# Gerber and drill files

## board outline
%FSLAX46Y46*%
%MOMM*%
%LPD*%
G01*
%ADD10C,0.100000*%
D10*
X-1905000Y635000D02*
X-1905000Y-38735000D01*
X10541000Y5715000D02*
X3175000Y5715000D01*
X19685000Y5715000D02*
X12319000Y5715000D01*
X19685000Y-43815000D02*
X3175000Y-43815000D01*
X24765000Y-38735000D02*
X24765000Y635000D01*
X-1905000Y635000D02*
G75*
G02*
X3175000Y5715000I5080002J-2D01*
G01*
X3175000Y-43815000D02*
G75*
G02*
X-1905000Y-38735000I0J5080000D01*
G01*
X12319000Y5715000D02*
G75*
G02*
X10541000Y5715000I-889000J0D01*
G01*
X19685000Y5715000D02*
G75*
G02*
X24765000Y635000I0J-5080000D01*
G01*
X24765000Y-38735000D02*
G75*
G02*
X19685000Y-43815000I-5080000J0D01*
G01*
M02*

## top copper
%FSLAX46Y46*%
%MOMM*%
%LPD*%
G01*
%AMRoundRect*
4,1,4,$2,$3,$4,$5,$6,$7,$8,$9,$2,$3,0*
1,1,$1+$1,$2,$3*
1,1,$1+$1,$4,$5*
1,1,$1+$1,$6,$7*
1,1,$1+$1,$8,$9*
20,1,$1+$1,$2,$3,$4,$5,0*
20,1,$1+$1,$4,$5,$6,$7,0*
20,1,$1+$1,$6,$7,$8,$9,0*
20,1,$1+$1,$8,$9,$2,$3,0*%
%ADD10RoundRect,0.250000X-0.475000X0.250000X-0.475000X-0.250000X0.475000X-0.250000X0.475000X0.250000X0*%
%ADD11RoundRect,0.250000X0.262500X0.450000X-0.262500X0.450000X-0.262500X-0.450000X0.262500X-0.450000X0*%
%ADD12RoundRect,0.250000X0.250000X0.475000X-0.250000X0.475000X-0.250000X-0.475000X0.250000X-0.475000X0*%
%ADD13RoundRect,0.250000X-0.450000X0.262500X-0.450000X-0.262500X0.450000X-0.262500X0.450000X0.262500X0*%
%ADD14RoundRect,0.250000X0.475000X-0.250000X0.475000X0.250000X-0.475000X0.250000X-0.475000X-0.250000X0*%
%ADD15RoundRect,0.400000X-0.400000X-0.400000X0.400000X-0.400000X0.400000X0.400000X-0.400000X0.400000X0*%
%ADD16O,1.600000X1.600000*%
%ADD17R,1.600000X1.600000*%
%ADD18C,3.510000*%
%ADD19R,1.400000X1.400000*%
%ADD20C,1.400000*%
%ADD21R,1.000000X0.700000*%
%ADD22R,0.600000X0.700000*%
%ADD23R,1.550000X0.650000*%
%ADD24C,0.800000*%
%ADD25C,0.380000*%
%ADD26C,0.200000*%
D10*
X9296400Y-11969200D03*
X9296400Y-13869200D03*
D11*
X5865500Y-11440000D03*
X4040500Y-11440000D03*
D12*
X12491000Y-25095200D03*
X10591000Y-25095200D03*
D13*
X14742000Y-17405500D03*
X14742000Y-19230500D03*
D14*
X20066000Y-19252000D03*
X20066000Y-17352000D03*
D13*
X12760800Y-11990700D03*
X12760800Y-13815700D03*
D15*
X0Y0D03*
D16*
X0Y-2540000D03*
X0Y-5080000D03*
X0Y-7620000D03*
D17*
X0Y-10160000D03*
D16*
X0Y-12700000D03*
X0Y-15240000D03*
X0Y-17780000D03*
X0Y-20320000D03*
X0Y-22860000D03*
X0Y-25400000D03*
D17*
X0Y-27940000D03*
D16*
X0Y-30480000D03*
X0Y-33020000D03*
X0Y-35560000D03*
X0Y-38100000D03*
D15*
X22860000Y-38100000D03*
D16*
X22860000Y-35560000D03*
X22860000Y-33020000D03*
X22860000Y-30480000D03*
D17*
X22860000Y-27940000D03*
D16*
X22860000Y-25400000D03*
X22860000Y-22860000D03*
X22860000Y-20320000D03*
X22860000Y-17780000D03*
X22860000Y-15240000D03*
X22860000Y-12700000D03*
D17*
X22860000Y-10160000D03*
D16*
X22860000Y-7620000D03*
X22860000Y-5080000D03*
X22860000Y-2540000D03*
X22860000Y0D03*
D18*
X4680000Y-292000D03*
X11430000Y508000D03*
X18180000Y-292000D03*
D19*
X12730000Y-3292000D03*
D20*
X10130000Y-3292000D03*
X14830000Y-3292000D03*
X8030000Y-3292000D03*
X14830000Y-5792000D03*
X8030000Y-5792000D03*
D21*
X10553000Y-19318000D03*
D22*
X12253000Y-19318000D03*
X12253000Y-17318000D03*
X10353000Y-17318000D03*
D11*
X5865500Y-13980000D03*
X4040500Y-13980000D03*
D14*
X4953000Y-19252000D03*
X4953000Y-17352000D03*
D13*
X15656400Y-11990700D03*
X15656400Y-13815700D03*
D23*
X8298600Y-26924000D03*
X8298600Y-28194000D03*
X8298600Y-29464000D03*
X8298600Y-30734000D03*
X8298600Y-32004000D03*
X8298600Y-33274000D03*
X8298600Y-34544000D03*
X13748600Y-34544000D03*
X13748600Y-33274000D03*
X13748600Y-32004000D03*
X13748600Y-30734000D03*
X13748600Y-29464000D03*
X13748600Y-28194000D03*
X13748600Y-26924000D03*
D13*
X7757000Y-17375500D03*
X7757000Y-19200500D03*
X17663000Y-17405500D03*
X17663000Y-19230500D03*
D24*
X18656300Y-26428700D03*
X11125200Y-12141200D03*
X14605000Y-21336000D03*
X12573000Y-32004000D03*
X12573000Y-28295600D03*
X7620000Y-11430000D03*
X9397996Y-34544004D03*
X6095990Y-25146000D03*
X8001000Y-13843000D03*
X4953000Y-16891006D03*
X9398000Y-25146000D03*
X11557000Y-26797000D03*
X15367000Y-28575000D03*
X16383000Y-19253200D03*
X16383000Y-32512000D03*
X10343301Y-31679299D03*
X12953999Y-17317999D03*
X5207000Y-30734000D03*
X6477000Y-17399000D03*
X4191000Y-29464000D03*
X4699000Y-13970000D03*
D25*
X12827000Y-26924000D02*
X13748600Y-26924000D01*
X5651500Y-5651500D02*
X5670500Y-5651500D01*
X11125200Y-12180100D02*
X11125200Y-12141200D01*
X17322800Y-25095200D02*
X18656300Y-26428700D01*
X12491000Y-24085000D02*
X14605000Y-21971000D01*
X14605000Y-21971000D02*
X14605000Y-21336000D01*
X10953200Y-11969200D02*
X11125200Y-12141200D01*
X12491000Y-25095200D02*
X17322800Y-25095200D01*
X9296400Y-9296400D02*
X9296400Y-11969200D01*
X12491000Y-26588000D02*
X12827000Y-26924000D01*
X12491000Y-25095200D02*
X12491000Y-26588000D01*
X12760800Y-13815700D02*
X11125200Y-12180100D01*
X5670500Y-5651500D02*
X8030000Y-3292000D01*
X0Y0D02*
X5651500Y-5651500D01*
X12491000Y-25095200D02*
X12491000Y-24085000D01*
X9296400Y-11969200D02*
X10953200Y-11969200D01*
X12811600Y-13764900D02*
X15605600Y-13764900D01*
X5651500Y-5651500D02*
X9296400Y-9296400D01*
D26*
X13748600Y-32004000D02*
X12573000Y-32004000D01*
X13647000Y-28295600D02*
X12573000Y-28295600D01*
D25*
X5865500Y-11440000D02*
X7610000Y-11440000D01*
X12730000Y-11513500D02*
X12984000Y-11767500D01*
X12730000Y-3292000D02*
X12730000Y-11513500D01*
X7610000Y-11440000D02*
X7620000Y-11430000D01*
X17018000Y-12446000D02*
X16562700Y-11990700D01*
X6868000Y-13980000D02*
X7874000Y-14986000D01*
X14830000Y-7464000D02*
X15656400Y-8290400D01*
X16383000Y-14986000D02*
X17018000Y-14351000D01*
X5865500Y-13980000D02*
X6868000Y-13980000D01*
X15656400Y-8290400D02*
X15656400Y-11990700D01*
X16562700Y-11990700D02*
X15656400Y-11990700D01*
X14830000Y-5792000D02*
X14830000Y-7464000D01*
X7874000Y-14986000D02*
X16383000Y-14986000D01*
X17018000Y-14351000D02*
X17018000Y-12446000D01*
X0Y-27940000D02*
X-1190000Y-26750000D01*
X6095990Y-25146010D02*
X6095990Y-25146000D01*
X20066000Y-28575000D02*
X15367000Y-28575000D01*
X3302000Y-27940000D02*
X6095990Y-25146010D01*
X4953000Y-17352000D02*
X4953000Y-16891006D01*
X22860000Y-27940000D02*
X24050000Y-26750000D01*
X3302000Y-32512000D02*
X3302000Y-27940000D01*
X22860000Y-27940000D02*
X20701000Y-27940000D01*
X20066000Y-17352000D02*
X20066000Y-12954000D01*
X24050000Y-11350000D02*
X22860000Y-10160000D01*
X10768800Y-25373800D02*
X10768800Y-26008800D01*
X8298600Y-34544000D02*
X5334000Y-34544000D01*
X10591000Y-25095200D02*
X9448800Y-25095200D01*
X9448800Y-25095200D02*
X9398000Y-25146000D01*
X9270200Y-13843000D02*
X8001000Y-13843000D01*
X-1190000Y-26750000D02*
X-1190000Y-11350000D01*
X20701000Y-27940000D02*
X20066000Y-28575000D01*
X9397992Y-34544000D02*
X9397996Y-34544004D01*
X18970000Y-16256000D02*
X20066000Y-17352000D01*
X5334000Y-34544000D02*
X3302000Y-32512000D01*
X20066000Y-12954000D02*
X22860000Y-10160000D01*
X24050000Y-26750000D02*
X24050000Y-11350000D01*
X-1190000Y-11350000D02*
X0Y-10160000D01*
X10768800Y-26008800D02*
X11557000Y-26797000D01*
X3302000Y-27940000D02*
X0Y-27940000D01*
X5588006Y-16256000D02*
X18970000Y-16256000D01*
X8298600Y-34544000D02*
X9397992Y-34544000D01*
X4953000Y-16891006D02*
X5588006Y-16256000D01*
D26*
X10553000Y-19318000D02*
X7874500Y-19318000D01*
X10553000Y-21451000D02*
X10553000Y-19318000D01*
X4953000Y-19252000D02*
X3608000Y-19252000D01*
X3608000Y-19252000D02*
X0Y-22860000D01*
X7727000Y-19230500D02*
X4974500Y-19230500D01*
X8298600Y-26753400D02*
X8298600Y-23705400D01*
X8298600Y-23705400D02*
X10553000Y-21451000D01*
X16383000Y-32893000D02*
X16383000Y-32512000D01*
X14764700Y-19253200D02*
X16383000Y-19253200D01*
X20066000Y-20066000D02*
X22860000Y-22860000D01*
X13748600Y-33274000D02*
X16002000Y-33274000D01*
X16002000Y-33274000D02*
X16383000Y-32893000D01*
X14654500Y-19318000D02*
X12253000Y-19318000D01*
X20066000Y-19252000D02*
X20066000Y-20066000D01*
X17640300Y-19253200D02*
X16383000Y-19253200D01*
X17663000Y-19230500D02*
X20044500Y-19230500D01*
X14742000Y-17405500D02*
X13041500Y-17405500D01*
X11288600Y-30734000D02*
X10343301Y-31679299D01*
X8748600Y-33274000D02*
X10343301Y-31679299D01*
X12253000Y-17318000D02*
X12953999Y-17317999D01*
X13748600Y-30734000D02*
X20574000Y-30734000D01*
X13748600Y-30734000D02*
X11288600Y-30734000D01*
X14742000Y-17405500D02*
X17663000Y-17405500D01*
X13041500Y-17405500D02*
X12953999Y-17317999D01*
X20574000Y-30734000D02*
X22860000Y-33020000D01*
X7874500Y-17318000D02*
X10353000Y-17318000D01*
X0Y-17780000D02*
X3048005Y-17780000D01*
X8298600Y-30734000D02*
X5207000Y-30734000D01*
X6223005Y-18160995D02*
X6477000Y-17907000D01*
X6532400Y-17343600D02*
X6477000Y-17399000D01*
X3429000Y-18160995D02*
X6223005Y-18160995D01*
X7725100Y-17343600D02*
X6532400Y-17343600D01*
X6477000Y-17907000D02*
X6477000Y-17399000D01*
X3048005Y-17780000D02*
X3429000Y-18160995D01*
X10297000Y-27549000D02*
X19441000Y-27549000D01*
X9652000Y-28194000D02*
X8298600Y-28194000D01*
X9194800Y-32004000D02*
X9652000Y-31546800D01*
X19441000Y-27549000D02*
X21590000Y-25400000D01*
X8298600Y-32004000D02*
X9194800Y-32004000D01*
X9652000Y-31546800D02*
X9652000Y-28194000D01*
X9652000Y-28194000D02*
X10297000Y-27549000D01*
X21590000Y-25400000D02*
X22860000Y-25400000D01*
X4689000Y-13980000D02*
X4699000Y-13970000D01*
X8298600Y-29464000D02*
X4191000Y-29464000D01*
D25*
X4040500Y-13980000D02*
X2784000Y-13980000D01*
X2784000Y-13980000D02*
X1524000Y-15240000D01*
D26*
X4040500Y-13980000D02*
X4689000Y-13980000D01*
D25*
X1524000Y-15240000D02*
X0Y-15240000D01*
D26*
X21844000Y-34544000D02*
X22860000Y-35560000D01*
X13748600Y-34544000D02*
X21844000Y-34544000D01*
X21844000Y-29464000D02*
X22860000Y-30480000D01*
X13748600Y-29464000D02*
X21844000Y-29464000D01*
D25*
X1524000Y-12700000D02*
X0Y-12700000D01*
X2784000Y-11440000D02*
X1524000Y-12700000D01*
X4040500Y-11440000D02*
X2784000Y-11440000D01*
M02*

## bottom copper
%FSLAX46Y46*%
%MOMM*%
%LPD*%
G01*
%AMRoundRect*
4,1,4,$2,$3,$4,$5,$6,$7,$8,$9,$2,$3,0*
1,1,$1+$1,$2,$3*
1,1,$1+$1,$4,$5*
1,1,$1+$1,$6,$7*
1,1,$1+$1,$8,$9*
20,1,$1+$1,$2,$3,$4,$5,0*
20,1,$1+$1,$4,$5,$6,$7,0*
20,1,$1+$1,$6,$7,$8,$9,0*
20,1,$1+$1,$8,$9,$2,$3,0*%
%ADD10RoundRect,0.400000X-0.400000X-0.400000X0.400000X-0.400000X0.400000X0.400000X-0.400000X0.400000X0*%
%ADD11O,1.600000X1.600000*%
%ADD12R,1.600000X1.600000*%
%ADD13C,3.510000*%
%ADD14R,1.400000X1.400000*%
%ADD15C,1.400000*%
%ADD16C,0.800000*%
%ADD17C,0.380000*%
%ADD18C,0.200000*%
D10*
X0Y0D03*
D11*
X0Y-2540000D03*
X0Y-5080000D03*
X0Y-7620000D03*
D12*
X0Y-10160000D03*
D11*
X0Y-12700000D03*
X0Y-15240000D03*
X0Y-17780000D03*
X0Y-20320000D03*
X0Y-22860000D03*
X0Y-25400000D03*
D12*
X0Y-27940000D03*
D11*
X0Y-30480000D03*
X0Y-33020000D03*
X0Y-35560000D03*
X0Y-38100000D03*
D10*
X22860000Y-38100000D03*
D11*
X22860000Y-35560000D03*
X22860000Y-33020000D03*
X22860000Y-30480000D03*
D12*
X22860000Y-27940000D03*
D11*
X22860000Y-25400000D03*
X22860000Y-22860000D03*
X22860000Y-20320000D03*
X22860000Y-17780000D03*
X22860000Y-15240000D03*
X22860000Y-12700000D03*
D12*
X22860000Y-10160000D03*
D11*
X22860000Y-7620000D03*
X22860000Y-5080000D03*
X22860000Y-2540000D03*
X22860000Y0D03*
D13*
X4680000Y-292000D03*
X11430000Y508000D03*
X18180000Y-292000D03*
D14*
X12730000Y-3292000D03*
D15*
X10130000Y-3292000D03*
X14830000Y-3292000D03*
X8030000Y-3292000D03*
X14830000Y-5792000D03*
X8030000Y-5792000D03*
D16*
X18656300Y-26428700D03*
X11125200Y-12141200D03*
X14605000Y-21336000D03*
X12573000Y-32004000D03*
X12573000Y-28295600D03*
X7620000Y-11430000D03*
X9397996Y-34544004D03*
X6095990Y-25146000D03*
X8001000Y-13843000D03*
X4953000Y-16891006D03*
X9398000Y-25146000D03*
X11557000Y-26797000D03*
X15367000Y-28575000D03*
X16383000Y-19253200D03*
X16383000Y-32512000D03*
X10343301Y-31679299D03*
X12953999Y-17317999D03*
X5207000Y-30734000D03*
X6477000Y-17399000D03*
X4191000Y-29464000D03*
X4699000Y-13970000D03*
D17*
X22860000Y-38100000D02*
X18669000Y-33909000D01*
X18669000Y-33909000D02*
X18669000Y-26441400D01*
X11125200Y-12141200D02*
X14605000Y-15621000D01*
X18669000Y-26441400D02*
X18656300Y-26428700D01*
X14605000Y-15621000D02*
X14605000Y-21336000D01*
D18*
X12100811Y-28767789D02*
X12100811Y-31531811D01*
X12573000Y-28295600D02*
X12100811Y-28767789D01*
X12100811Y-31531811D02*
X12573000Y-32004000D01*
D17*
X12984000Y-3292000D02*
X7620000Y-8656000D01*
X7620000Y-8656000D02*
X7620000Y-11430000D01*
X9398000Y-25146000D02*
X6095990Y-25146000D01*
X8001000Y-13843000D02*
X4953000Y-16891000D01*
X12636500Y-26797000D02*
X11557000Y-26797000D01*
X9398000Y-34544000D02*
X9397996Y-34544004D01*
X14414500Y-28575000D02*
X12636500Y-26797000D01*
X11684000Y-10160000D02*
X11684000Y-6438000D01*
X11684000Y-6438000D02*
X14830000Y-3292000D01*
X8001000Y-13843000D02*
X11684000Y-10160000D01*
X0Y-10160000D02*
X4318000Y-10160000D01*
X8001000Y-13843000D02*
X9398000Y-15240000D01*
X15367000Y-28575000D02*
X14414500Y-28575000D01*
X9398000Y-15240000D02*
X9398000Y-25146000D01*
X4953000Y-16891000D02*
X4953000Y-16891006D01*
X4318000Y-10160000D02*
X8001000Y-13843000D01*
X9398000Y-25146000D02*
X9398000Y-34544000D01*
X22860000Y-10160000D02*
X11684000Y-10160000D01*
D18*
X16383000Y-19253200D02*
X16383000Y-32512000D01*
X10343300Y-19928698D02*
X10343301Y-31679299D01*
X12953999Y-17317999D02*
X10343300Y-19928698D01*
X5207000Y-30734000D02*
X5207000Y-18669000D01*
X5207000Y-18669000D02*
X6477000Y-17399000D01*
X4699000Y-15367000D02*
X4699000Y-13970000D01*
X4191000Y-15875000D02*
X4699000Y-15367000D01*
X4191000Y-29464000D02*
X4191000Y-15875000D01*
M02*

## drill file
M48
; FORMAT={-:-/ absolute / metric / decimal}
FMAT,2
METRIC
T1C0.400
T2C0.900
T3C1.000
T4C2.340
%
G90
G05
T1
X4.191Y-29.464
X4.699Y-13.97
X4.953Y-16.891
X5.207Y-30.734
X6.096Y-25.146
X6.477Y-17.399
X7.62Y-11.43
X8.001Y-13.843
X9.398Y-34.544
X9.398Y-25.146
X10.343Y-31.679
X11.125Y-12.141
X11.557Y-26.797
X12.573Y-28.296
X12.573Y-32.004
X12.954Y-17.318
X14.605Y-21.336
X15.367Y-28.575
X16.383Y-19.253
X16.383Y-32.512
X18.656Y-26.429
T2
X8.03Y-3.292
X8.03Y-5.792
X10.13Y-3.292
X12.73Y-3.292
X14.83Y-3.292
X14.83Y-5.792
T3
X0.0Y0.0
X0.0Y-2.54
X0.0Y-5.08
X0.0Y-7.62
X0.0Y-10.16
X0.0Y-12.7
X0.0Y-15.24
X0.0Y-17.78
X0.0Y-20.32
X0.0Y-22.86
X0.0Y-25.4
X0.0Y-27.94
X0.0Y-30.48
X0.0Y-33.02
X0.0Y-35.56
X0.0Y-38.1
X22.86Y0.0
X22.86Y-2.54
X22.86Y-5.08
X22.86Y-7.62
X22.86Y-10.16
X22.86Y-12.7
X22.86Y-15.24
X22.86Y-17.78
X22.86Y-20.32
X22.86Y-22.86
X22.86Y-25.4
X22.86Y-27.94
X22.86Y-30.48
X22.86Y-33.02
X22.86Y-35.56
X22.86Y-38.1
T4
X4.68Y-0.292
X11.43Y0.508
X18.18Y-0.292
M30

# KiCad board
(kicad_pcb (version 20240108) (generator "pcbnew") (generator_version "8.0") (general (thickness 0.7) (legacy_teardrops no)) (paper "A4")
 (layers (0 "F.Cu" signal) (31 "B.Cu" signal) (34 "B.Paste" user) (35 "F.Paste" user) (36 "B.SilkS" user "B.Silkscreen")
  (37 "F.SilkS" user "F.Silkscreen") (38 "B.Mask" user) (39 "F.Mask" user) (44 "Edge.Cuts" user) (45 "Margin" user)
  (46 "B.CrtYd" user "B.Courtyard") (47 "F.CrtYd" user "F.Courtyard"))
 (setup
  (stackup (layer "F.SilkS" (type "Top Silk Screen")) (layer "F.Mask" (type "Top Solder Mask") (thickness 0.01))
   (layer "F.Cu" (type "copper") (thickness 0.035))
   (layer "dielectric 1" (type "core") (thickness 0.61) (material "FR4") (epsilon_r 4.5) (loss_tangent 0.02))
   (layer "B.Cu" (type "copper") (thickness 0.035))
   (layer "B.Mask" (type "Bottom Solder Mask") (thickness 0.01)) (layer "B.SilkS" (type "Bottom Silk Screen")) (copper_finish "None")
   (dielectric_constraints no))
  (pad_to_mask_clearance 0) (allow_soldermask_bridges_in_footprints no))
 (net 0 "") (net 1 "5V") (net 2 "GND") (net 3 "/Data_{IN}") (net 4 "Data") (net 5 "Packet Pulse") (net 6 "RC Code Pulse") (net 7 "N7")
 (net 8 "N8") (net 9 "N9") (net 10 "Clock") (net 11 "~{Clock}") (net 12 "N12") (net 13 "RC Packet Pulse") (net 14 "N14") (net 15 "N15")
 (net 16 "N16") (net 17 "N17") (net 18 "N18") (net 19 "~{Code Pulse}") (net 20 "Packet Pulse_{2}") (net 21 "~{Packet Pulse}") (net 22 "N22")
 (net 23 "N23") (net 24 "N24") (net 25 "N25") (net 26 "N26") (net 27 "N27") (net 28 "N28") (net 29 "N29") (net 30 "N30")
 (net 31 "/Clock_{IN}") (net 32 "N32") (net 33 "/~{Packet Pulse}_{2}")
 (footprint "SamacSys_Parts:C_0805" (layer "F.Cu") (at 9.2964 12.9032 180)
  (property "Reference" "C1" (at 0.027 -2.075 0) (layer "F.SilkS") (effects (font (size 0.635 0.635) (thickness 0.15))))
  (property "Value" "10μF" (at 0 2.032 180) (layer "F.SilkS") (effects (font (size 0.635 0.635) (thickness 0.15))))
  (pad "1" smd roundrect (at 0 0.934 270) (size 1 1.45) (layers "F.Cu" "F.Paste" "F.Mask") (roundrect_rratio 0.25) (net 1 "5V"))
  (pad "2" smd roundrect (at 0 -0.966 270) (size 1 1.45) (layers "F.Cu" "F.Paste" "F.Mask") (roundrect_rratio 0.25) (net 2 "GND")))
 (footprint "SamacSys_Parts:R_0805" (layer "F.Cu") (at 4.953 11.43 90)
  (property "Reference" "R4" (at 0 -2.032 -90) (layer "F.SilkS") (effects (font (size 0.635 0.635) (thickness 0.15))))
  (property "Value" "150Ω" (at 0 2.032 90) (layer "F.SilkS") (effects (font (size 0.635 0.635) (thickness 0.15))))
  (pad "1" smd roundrect (at -0.01 0.9125 180) (size 1.025 1.4) (layers "F.Cu" "F.Paste" "F.Mask") (roundrect_rratio 0.243902)
   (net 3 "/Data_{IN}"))
  (pad "2" smd roundrect (at -0.01 -0.9125 180) (size 1.025 1.4) (layers "F.Cu" "F.Paste" "F.Mask") (roundrect_rratio 0.243902)
   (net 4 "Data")))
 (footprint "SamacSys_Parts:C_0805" (layer "F.Cu") (at 11.557 25.0952 90)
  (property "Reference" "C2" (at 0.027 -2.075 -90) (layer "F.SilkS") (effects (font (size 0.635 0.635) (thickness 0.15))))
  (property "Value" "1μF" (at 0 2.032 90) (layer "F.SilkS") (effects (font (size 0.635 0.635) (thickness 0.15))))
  (pad "1" smd roundrect (at 0 0.934 180) (size 1 1.45) (layers "F.Cu" "F.Paste" "F.Mask") (roundrect_rratio 0.25) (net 1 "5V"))
  (pad "2" smd roundrect (at 0 -0.966 180) (size 1 1.45) (layers "F.Cu" "F.Paste" "F.Mask") (roundrect_rratio 0.25) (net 2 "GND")))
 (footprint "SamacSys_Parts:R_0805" (layer "F.Cu") (at 14.732 18.318 180)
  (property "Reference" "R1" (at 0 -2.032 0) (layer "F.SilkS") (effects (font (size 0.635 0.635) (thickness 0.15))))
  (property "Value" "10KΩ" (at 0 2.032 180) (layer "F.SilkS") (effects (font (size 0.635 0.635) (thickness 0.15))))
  (pad "1" smd roundrect (at -0.01 0.9125 270) (size 1.025 1.4) (layers "F.Cu" "F.Paste" "F.Mask") (roundrect_rratio 0.243902)
   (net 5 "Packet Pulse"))
  (pad "2" smd roundrect (at -0.01 -0.9125 270) (size 1.025 1.4) (layers "F.Cu" "F.Paste" "F.Mask") (roundrect_rratio 0.243902)
   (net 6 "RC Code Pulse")))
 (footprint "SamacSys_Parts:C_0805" (layer "F.Cu") (at 20.066 18.318)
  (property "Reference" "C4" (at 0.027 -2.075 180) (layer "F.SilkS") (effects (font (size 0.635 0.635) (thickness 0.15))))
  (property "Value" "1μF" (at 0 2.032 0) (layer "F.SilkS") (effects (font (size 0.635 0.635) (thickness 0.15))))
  (pad "1" smd roundrect (at 0 0.934 90) (size 1 1.45) (layers "F.Cu" "F.Paste" "F.Mask") (roundrect_rratio 0.25) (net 6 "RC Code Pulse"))
  (pad "2" smd roundrect (at 0 -0.966 90) (size 1 1.45) (layers "F.Cu" "F.Paste" "F.Mask") (roundrect_rratio 0.25) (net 2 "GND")))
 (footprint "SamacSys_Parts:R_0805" (layer "F.Cu") (at 12.7508 12.9032 180)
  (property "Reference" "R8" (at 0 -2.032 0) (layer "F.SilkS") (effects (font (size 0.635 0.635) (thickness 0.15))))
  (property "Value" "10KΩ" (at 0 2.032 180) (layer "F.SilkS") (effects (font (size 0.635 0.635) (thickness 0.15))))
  (pad "1" smd roundrect (at -0.01 0.9125 270) (size 1.025 1.4) (layers "F.Cu" "F.Paste" "F.Mask") (roundrect_rratio 0.243902)
   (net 3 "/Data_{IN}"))
  (pad "2" smd roundrect (at -0.01 -0.9125 270) (size 1.025 1.4) (layers "F.Cu" "F.Paste" "F.Mask") (roundrect_rratio 0.243902) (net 1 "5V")))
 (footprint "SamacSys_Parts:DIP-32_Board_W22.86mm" (layer "F.Cu") (at 0 0)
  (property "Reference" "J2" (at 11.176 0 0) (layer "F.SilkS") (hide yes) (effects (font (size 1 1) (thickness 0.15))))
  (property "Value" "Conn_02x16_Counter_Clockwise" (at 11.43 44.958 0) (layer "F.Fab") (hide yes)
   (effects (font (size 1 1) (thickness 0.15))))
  (fp_line (start -1.905 -0.635) (end -1.905 38.735) (stroke (width 0.1) (type solid)) (layer "Edge.Cuts"))
  (fp_line (start 10.541 -5.715) (end 3.175 -5.715) (stroke (width 0.1) (type solid)) (layer "Edge.Cuts"))
  (fp_line (start 19.685 -5.715) (end 12.319 -5.715) (stroke (width 0.1) (type solid)) (layer "Edge.Cuts"))
  (fp_line (start 19.685 43.815) (end 3.175 43.815) (stroke (width 0.1) (type solid)) (layer "Edge.Cuts"))
  (fp_line (start 24.765 38.735) (end 24.765 -0.635) (stroke (width 0.1) (type solid)) (layer "Edge.Cuts"))
  (fp_arc (start -1.905 -0.635) (mid -0.417102 -4.227102) (end 3.175 -5.715) (stroke (width 0.1) (type solid)) (layer "Edge.Cuts"))
  (fp_arc (start 3.175 43.815) (mid -0.417102 42.327102) (end -1.905 38.735) (stroke (width 0.1) (type solid)) (layer "Edge.Cuts"))
  (fp_arc (start 12.319 -5.715) (mid 11.43 -4.826) (end 10.541 -5.715) (stroke (width 0.1) (type default)) (layer "Edge.Cuts"))
  (fp_arc (start 19.685 -5.715) (mid 23.277102 -4.227102) (end 24.765 -0.635) (stroke (width 0.1) (type solid)) (layer "Edge.Cuts"))
  (fp_arc (start 24.765 38.735) (mid 23.277102 42.327102) (end 19.685 43.815) (stroke (width 0.1) (type solid)) (layer "Edge.Cuts"))
  (pad "1" thru_hole roundrect (at 0 0) (size 1.6 1.6) (drill 1) (layers "*.Cu" "*.Mask") (remove_unused_layers no) (roundrect_rratio 0.25)
   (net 1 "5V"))
  (pad "2" thru_hole oval (at 0 2.54) (size 1.6 1.6) (drill 1) (layers "*.Cu" "*.Mask") (remove_unused_layers no) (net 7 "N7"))
  (pad "3" thru_hole oval (at 0 5.08) (size 1.6 1.6) (drill 1) (layers "*.Cu" "*.Mask") (remove_unused_layers no) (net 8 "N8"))
  (pad "4" thru_hole oval (at 0 7.62) (size 1.6 1.6) (drill 1) (layers "*.Cu" "*.Mask") (remove_unused_layers no) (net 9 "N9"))
  (pad "5" thru_hole rect (at 0 10.16) (size 1.6 1.6) (drill 1) (layers "*.Cu" "*.Mask") (remove_unused_layers no) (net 2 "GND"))
  (pad "6" thru_hole oval (at 0 12.7) (size 1.6 1.6) (drill 1) (layers "*.Cu" "*.Mask") (remove_unused_layers no) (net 4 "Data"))
  (pad "7" thru_hole oval (at 0 15.24) (size 1.6 1.6) (drill 1) (layers "*.Cu" "*.Mask") (remove_unused_layers no) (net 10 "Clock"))
  (pad "8" thru_hole oval (at 0 17.78) (size 1.6 1.6) (drill 1) (layers "*.Cu" "*.Mask") (remove_unused_layers no) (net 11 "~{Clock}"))
  (pad "9" thru_hole oval (at 0 20.32) (size 1.6 1.6) (drill 1) (layers "*.Cu" "*.Mask") (remove_unused_layers no) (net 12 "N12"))
  (pad "10" thru_hole oval (at 0 22.86) (size 1.6 1.6) (drill 1) (layers "*.Cu" "*.Mask") (remove_unused_layers no)
   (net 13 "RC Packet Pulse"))
  (pad "11" thru_hole oval (at 0 25.4) (size 1.6 1.6) (drill 1) (layers "*.Cu" "*.Mask") (remove_unused_layers no) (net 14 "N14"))
  (pad "12" thru_hole rect (at 0 27.94) (size 1.6 1.6) (drill 1) (layers "*.Cu" "*.Mask") (remove_unused_layers no) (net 2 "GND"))
  (pad "13" thru_hole oval (at 0 30.48) (size 1.6 1.6) (drill 1) (layers "*.Cu" "*.Mask") (remove_unused_layers no) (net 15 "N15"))
  (pad "14" thru_hole oval (at 0 33.02) (size 1.6 1.6) (drill 1) (layers "*.Cu" "*.Mask") (remove_unused_layers no) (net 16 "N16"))
  (pad "15" thru_hole oval (at 0 35.56) (size 1.6 1.6) (drill 1) (layers "*.Cu" "*.Mask") (remove_unused_layers no) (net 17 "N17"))
  (pad "16" thru_hole oval (at 0 38.1) (size 1.6 1.6) (drill 1) (layers "*.Cu" "*.Mask") (remove_unused_layers no) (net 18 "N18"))
  (pad "17" thru_hole roundrect (at 22.86 38.1) (size 1.6 1.6) (drill 1) (layers "*.Cu" "*.Mask") (remove_unused_layers no)
   (roundrect_rratio 0.25) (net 1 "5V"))
  (pad "18" thru_hole oval (at 22.86 35.56) (size 1.6 1.6) (drill 1) (layers "*.Cu" "*.Mask") (remove_unused_layers no)
   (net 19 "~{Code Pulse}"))
  (pad "19" thru_hole oval (at 22.86 33.02) (size 1.6 1.6) (drill 1) (layers "*.Cu" "*.Mask") (remove_unused_layers no)
   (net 5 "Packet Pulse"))
  (pad "20" thru_hole oval (at 22.86 30.48) (size 1.6 1.6) (drill 1) (layers "*.Cu" "*.Mask") (remove_unused_layers no)
   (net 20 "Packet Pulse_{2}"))
  (pad "21" thru_hole rect (at 22.86 27.94) (size 1.6 1.6) (drill 1) (layers "*.Cu" "*.Mask") (remove_unused_layers no) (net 2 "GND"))
  (pad "22" thru_hole oval (at 22.86 25.4) (size 1.6 1.6) (drill 1) (layers "*.Cu" "*.Mask") (remove_unused_layers no)
   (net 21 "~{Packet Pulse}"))
  (pad "23" thru_hole oval (at 22.86 22.86) (size 1.6 1.6) (drill 1) (layers "*.Cu" "*.Mask") (remove_unused_layers no)
   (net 6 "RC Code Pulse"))
  (pad "24" thru_hole oval (at 22.86 20.32) (size 1.6 1.6) (drill 1) (layers "*.Cu" "*.Mask") (remove_unused_layers no) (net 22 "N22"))
  (pad "25" thru_hole oval (at 22.86 17.78) (size 1.6 1.6) (drill 1) (layers "*.Cu" "*.Mask") (remove_unused_layers no) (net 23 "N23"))
  (pad "26" thru_hole oval (at 22.86 15.24) (size 1.6 1.6) (drill 1) (layers "*.Cu" "*.Mask") (remove_unused_layers no) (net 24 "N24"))
  (pad "27" thru_hole oval (at 22.86 12.7) (size 1.6 1.6) (drill 1) (layers "*.Cu" "*.Mask") (remove_unused_layers no) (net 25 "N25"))
  (pad "28" thru_hole rect (at 22.86 10.16) (size 1.6 1.6) (drill 1) (layers "*.Cu" "*.Mask") (remove_unused_layers no) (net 2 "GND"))
  (pad "29" thru_hole oval (at 22.86 7.62) (size 1.6 1.6) (drill 1) (layers "*.Cu" "*.Mask") (remove_unused_layers no) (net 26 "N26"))
  (pad "30" thru_hole oval (at 22.86 5.08) (size 1.6 1.6) (drill 1) (layers "*.Cu" "*.Mask") (remove_unused_layers no) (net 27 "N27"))
  (pad "31" thru_hole oval (at 22.86 2.54) (size 1.6 1.6) (drill 1) (layers "*.Cu" "*.Mask") (remove_unused_layers no) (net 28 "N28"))
  (pad "32" thru_hole oval (at 22.86 0) (size 1.6 1.6) (drill 1) (layers "*.Cu" "*.Mask") (remove_unused_layers no) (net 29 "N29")))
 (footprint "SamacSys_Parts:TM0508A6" (layer "F.Cu") (at 12.73 3.292)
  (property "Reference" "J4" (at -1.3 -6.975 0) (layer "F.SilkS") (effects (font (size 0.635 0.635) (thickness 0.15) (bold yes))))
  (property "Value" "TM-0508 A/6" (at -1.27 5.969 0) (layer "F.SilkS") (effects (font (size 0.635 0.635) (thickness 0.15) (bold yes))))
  (pad "" thru_hole circle (at -8.05 -3) (size 3.51 3.51) (drill 2.34) (layers "*.Cu" "*.Mask") (remove_unused_layers no))
  (pad "" thru_hole circle (at -1.3 -3.8) (size 3.51 3.51) (drill 2.34) (layers "*.Cu" "*.Mask") (remove_unused_layers no))
  (pad "" thru_hole circle (at 5.45 -3) (size 3.51 3.51) (drill 2.34) (layers "*.Cu" "*.Mask") (remove_unused_layers no))
  (pad "1" thru_hole rect (at 0 0) (size 1.4 1.4) (drill 0.9) (layers "*.Cu" "*.Mask") (remove_unused_layers no) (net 3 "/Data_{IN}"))
  (pad "2" thru_hole circle (at -2.6 0) (size 1.4 1.4) (drill 0.9) (layers "*.Cu" "*.Mask") (remove_unused_layers no) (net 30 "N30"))
  (pad "3" thru_hole circle (at 2.1 0) (size 1.4 1.4) (drill 0.9) (layers "*.Cu" "*.Mask") (remove_unused_layers no) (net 2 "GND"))
  (pad "4" thru_hole circle (at -4.7 0) (size 1.4 1.4) (drill 0.9) (layers "*.Cu" "*.Mask") (remove_unused_layers no) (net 1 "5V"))
  (pad "5" thru_hole circle (at 2.1 2.5) (size 1.4 1.4) (drill 0.9) (layers "*.Cu" "*.Mask") (remove_unused_layers no)
   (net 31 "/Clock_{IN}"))
  (pad "6" thru_hole circle (at -4.7 2.5) (size 1.4 1.4) (drill 0.9) (layers "*.Cu" "*.Mask") (remove_unused_layers no) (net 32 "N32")))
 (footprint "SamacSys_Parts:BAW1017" (layer "F.Cu") (at 11.303 18.318)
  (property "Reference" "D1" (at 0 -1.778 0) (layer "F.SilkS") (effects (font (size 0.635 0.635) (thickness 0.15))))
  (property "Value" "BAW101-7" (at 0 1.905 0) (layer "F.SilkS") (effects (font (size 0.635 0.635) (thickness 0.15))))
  (pad "1" smd rect (at -0.75 1 90) (size 0.7 1) (layers "F.Cu" "F.Paste" "F.Mask") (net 13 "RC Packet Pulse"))
  (pad "2" smd rect (at 0.95 1) (size 0.6 0.7) (layers "F.Cu" "F.Paste" "F.Mask") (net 6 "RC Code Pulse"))
  (pad "3" smd rect (at 0.95 -1) (size 0.6 0.7) (layers "F.Cu" "F.Paste" "F.Mask") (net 5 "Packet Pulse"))
  (pad "4" smd rect (at -0.95 -1) (size 0.6 0.7) (layers "F.Cu" "F.Paste" "F.Mask") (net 11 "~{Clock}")))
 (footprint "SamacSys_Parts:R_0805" (layer "F.Cu") (at 4.953 13.97 90)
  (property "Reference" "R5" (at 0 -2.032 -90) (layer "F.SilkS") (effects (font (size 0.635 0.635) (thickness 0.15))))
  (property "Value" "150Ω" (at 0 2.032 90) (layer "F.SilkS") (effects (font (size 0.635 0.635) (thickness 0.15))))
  (pad "1" smd roundrect (at -0.01 0.9125 180) (size 1.025 1.4) (layers "F.Cu" "F.Paste" "F.Mask") (roundrect_rratio 0.243902)
   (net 31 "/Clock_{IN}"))
  (pad "2" smd roundrect (at -0.01 -0.9125 180) (size 1.025 1.4) (layers "F.Cu" "F.Paste" "F.Mask") (roundrect_rratio 0.243902)
   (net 10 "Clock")))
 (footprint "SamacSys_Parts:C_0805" (layer "F.Cu") (at 4.953 18.318)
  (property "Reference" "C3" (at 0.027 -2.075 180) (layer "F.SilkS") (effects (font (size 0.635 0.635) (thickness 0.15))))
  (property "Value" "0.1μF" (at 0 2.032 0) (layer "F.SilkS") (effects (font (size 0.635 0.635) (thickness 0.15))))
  (pad "1" smd roundrect (at 0 0.934 90) (size 1 1.45) (layers "F.Cu" "F.Paste" "F.Mask") (roundrect_rratio 0.25) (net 13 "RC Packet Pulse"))
  (pad "2" smd roundrect (at 0 -0.966 90) (size 1 1.45) (layers "F.Cu" "F.Paste" "F.Mask") (roundrect_rratio 0.25) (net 2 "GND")))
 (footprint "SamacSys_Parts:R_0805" (layer "F.Cu") (at 15.6464 12.9032 180)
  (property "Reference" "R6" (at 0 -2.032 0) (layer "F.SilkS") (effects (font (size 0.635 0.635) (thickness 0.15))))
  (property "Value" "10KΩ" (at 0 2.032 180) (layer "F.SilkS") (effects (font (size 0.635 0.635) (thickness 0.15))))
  (pad "1" smd roundrect (at -0.01 0.9125 270) (size 1.025 1.4) (layers "F.Cu" "F.Paste" "F.Mask") (roundrect_rratio 0.243902)
   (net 31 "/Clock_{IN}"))
  (pad "2" smd roundrect (at -0.01 -0.9125 270) (size 1.025 1.4) (layers "F.Cu" "F.Paste" "F.Mask") (roundrect_rratio 0.243902) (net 1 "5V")))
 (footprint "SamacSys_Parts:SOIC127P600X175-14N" (layer "F.Cu") (at 11.0236 30.734)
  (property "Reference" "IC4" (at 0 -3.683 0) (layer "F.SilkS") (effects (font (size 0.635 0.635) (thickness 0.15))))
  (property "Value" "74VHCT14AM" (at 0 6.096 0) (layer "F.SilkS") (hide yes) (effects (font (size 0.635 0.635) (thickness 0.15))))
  (pad "1" smd rect (at -2.725 -3.81 90) (size 0.65 1.55) (layers "F.Cu" "F.Paste" "F.Mask") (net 13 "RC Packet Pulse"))
  (pad "2" smd rect (at -2.725 -2.54 90) (size 0.65 1.55) (layers "F.Cu" "F.Paste" "F.Mask") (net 21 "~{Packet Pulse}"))
  (pad "3" smd rect (at -2.725 -1.27 90) (size 0.65 1.55) (layers "F.Cu" "F.Paste" "F.Mask") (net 10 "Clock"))
  (pad "4" smd rect (at -2.725 0 90) (size 0.65 1.55) (layers "F.Cu" "F.Paste" "F.Mask") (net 11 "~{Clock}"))
  (pad "5" smd rect (at -2.725 1.27 90) (size 0.65 1.55) (layers "F.Cu" "F.Paste" "F.Mask") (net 21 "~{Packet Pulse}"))
  (pad "6" smd rect (at -2.725 2.54 90) (size 0.65 1.55) (layers "F.Cu" "F.Paste" "F.Mask") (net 5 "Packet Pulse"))
  (pad "7" smd rect (at -2.725 3.81 90) (size 0.65 1.55) (layers "F.Cu" "F.Paste" "F.Mask") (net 2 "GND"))
  (pad "8" smd rect (at 2.725 3.81 90) (size 0.65 1.55) (layers "F.Cu" "F.Paste" "F.Mask") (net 19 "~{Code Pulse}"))
  (pad "9" smd rect (at 2.725 2.54 90) (size 0.65 1.55) (layers "F.Cu" "F.Paste" "F.Mask") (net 6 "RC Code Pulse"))
  (pad "10" smd rect (at 2.725 1.27 90) (size 0.65 1.55) (layers "F.Cu" "F.Paste" "F.Mask") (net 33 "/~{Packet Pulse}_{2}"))
  (pad "11" smd rect (at 2.725 0 90) (size 0.65 1.55) (layers "F.Cu" "F.Paste" "F.Mask") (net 5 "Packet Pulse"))
  (pad "12" smd rect (at 2.725 -1.27 90) (size 0.65 1.55) (layers "F.Cu" "F.Paste" "F.Mask") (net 20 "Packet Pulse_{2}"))
  (pad "13" smd rect (at 2.725 -2.54 90) (size 0.65 1.55) (layers "F.Cu" "F.Paste" "F.Mask") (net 33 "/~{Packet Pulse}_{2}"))
  (pad "14" smd rect (at 2.725 -3.81 90) (size 0.65 1.55) (layers "F.Cu" "F.Paste" "F.Mask") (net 1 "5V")))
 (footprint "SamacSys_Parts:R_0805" (layer "F.Cu") (at 7.747 18.288 180)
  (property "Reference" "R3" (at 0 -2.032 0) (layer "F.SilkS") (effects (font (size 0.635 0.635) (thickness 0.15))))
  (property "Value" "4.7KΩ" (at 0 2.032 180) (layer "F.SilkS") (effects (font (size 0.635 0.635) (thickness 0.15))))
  (pad "1" smd roundrect (at -0.01 0.9125 270) (size 1.025 1.4) (layers "F.Cu" "F.Paste" "F.Mask") (roundrect_rratio 0.243902)
   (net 11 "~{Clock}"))
  (pad "2" smd roundrect (at -0.01 -0.9125 270) (size 1.025 1.4) (layers "F.Cu" "F.Paste" "F.Mask") (roundrect_rratio 0.243902)
   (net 13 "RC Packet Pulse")))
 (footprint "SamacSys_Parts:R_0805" (layer "F.Cu") (at 17.653 18.318 180)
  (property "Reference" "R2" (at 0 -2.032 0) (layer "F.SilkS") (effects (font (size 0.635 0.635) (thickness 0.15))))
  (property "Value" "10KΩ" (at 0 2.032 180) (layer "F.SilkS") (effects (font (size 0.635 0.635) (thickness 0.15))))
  (pad "1" smd roundrect (at -0.01 0.9125 270) (size 1.025 1.4) (layers "F.Cu" "F.Paste" "F.Mask") (roundrect_rratio 0.243902)
   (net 5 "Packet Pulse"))
  (pad "2" smd roundrect (at -0.01 -0.9125 270) (size 1.025 1.4) (layers "F.Cu" "F.Paste" "F.Mask") (roundrect_rratio 0.243902)
   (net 6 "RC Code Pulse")))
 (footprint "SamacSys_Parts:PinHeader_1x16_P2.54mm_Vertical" (layer "B.Cu") (at 0 0 180)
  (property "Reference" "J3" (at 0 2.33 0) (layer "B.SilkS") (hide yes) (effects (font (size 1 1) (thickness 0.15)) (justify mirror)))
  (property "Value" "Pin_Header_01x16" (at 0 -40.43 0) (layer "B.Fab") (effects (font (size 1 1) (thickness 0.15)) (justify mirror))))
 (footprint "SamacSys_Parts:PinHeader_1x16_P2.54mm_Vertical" (layer "B.Cu") (at 22.86 0 180)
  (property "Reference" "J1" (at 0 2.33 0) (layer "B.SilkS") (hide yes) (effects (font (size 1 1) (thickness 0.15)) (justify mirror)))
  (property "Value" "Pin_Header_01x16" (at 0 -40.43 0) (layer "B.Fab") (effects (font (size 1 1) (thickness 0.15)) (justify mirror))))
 (segment (start 12.827 26.924) (end 13.7486 26.924) (width 0.38) (layer "F.Cu") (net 1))
 (segment (start 5.6515 5.6515) (end 5.6705 5.6515) (width 0.38) (layer "F.Cu") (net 1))
 (segment (start 11.1252 12.1801) (end 11.1252 12.1412) (width 0.38) (layer "F.Cu") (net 1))
 (segment (start 17.3228 25.0952) (end 18.6563 26.4287) (width 0.38) (layer "F.Cu") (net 1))
 (segment (start 12.491 24.085) (end 14.605 21.971) (width 0.38) (layer "F.Cu") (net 1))
 (segment (start 14.605 21.971) (end 14.605 21.336) (width 0.38) (layer "F.Cu") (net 1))
 (segment (start 10.9532 11.9692) (end 11.1252 12.1412) (width 0.38) (layer "F.Cu") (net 1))
 (segment (start 12.491 25.0952) (end 17.3228 25.0952) (width 0.38) (layer "F.Cu") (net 1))
 (segment (start 9.2964 9.2964) (end 9.2964 11.9692) (width 0.38) (layer "F.Cu") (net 1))
 (segment (start 12.491 26.588) (end 12.827 26.924) (width 0.38) (layer "F.Cu") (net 1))
 (segment (start 12.491 25.0952) (end 12.491 26.588) (width 0.38) (layer "F.Cu") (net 1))
 (segment (start 12.7608 13.8157) (end 11.1252 12.1801) (width 0.38) (layer "F.Cu") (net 1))
 (segment (start 5.6705 5.6515) (end 8.03 3.292) (width 0.38) (layer "F.Cu") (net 1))
 (segment (start 0 0) (end 5.6515 5.6515) (width 0.38) (layer "F.Cu") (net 1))
 (segment (start 12.491 25.0952) (end 12.491 24.085) (width 0.38) (layer "F.Cu") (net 1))
 (segment (start 9.2964 11.9692) (end 10.9532 11.9692) (width 0.38) (layer "F.Cu") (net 1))
 (segment (start 12.8116 13.7649) (end 15.6056 13.7649) (width 0.38) (layer "F.Cu") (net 1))
 (segment (start 5.6515 5.6515) (end 9.2964 9.2964) (width 0.38) (layer "F.Cu") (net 1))
 (via (at 18.6563 26.4287) (size 0.8) (drill 0.4) (layers "F.Cu" "B.Cu") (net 1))
 (via (at 11.1252 12.1412) (size 0.8) (drill 0.4) (layers "F.Cu" "B.Cu") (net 1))
 (via (at 14.605 21.336) (size 0.8) (drill 0.4) (layers "F.Cu" "B.Cu") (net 1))
 (segment (start 22.86 38.1) (end 18.669 33.909) (width 0.38) (layer "B.Cu") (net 1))
 (segment (start 18.669 33.909) (end 18.669 26.4414) (width 0.38) (layer "B.Cu") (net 1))
 (segment (start 11.1252 12.1412) (end 14.605 15.621) (width 0.38) (layer "B.Cu") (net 1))
 (segment (start 18.669 26.4414) (end 18.6563 26.4287) (width 0.38) (layer "B.Cu") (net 1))
 (segment (start 14.605 15.621) (end 14.605 21.336) (width 0.38) (layer "B.Cu") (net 1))
 (segment (start 13.7486 32.004) (end 12.573 32.004) (width 0.2) (layer "F.Cu") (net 33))
 (segment (start 13.647 28.2956) (end 12.573 28.2956) (width 0.2) (layer "F.Cu") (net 33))
 (via (at 12.573 32.004) (size 0.8) (drill 0.4) (layers "F.Cu" "B.Cu") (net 33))
 (via (at 12.573 28.2956) (size 0.8) (drill 0.4) (layers "F.Cu" "B.Cu") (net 33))
 (segment (start 12.100811 28.767789) (end 12.100811 31.531811) (width 0.2) (layer "B.Cu") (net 33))
 (segment (start 12.573 28.2956) (end 12.100811 28.767789) (width 0.2) (layer "B.Cu") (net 33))
 (segment (start 12.100811 31.531811) (end 12.573 32.004) (width 0.2) (layer "B.Cu") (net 33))
 (segment (start 5.8655 11.44) (end 7.61 11.44) (width 0.38) (layer "F.Cu") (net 3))
 (segment (start 12.73 11.5135) (end 12.984 11.7675) (width 0.38) (layer "F.Cu") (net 3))
 (segment (start 12.73 3.292) (end 12.73 11.5135) (width 0.38) (layer "F.Cu") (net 3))
 (segment (start 7.61 11.44) (end 7.62 11.43) (width 0.38) (layer "F.Cu") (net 3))
 (via (at 7.62 11.43) (size 0.8) (drill 0.4) (layers "F.Cu" "B.Cu") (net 3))
 (segment (start 12.984 3.292) (end 7.62 8.656) (width 0.38) (layer "B.Cu") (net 3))
 (segment (start 7.62 8.656) (end 7.62 11.43) (width 0.38) (layer "B.Cu") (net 3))
 (segment (start 17.018 12.446) (end 16.5627 11.9907) (width 0.38) (layer "F.Cu") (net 31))
 (segment (start 6.868 13.98) (end 7.874 14.986) (width 0.38) (layer "F.Cu") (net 31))
 (segment (start 14.83 7.464) (end 15.6564 8.2904) (width 0.38) (layer "F.Cu") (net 31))
 (segment (start 16.383 14.986) (end 17.018 14.351) (width 0.38) (layer "F.Cu") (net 31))
 (segment (start 5.8655 13.98) (end 6.868 13.98) (width 0.38) (layer "F.Cu") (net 31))
 (segment (start 15.6564 8.2904) (end 15.6564 11.9907) (width 0.38) (layer "F.Cu") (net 31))
 (segment (start 16.5627 11.9907) (end 15.6564 11.9907) (width 0.38) (layer "F.Cu") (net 31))
 (segment (start 14.83 5.792) (end 14.83 7.464) (width 0.38) (layer "F.Cu") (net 31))
 (segment (start 7.874 14.986) (end 16.383 14.986) (width 0.38) (layer "F.Cu") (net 31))
 (segment (start 17.018 14.351) (end 17.018 12.446) (width 0.38) (layer "F.Cu") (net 31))
 (segment (start 0 27.94) (end -1.19 26.75) (width 0.38) (layer "F.Cu") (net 2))
 (segment (start 6.09599 25.14601) (end 6.09599 25.146) (width 0.38) (layer "F.Cu") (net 2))
 (segment (start 20.066 28.575) (end 15.367 28.575) (width 0.38) (layer "F.Cu") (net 2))
 (segment (start 3.302 27.94) (end 6.09599 25.14601) (width 0.38) (layer "F.Cu") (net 2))
 (segment (start 4.953 17.352) (end 4.953 16.891006) (width 0.38) (layer "F.Cu") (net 2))
 (segment (start 22.86 27.94) (end 24.05 26.75) (width 0.38) (layer "F.Cu") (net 2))
 (segment (start 3.302 32.512) (end 3.302 27.94) (width 0.38) (layer "F.Cu") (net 2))
 (segment (start 22.86 27.94) (end 20.701 27.94) (width 0.38) (layer "F.Cu") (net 2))
 (segment (start 20.066 17.352) (end 20.066 12.954) (width 0.38) (layer "F.Cu") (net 2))
 (segment (start 24.05 11.35) (end 22.86 10.16) (width 0.38) (layer "F.Cu") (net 2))
 (segment (start 10.7688 25.3738) (end 10.7688 26.0088) (width 0.38) (layer "F.Cu") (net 2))
 (segment (start 8.2986 34.544) (end 5.334 34.544) (width 0.38) (layer "F.Cu") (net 2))
 (segment (start 10.591 25.0952) (end 9.4488 25.0952) (width 0.38) (layer "F.Cu") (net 2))
 (segment (start 9.4488 25.0952) (end 9.398 25.146) (width 0.38) (layer "F.Cu") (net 2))
 (segment (start 9.2702 13.843) (end 8.001 13.843) (width 0.38) (layer "F.Cu") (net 2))
 (segment (start -1.19 26.75) (end -1.19 11.35) (width 0.38) (layer "F.Cu") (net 2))
 (segment (start 20.701 27.94) (end 20.066 28.575) (width 0.38) (layer "F.Cu") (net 2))
 (segment (start 9.397992 34.544) (end 9.397996 34.544004) (width 0.38) (layer "F.Cu") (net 2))
 (segment (start 18.97 16.256) (end 20.066 17.352) (width 0.38) (layer "F.Cu") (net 2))
 (segment (start 5.334 34.544) (end 3.302 32.512) (width 0.38) (layer "F.Cu") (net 2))
 (segment (start 20.066 12.954) (end 22.86 10.16) (width 0.38) (layer "F.Cu") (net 2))
 (segment (start 24.05 26.75) (end 24.05 11.35) (width 0.38) (layer "F.Cu") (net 2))
 (segment (start -1.19 11.35) (end 0 10.16) (width 0.38) (layer "F.Cu") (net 2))
 (segment (start 10.7688 26.0088) (end 11.557 26.797) (width 0.38) (layer "F.Cu") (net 2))
 (segment (start 3.302 27.94) (end 0 27.94) (width 0.38) (layer "F.Cu") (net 2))
 (segment (start 5.588006 16.256) (end 18.97 16.256) (width 0.38) (layer "F.Cu") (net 2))
 (segment (start 8.2986 34.544) (end 9.397992 34.544) (width 0.38) (layer "F.Cu") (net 2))
 (segment (start 4.953 16.891006) (end 5.588006 16.256) (width 0.38) (layer "F.Cu") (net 2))
 (via (at 9.397996 34.544004) (size 0.8) (drill 0.4) (layers "F.Cu" "B.Cu") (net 2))
 (via (at 6.09599 25.146) (size 0.8) (drill 0.4) (layers "F.Cu" "B.Cu") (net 2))
 (via (at 8.001 13.843) (size 0.8) (drill 0.4) (layers "F.Cu" "B.Cu") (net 2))
 (via (at 4.953 16.891006) (size 0.8) (drill 0.4) (layers "F.Cu" "B.Cu") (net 2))
 (via (at 9.398 25.146) (size 0.8) (drill 0.4) (layers "F.Cu" "B.Cu") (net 2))
 (via (at 11.557 26.797) (size 0.8) (drill 0.4) (layers "F.Cu" "B.Cu") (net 2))
 (via (at 15.367 28.575) (size 0.8) (drill 0.4) (layers "F.Cu" "B.Cu") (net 2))
 (segment (start 9.398 25.146) (end 6.09599 25.146) (width 0.38) (layer "B.Cu") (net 2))
 (segment (start 8.001 13.843) (end 4.953 16.891) (width 0.38) (layer "B.Cu") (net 2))
 (segment (start 12.6365 26.797) (end 11.557 26.797) (width 0.38) (layer "B.Cu") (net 2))
 (segment (start 9.398 34.544) (end 9.397996 34.544004) (width 0.38) (layer "B.Cu") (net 2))
 (segment (start 14.4145 28.575) (end 12.6365 26.797) (width 0.38) (layer "B.Cu") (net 2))
 (segment (start 11.684 10.16) (end 11.684 6.438) (width 0.38) (layer "B.Cu") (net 2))
 (segment (start 11.684 6.438) (end 14.83 3.292) (width 0.38) (layer "B.Cu") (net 2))
 (segment (start 8.001 13.843) (end 11.684 10.16) (width 0.38) (layer "B.Cu") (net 2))
 (segment (start 0 10.16) (end 4.318 10.16) (width 0.38) (layer "B.Cu") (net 2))
 (segment (start 8.001 13.843) (end 9.398 15.24) (width 0.38) (layer "B.Cu") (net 2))
 (segment (start 15.367 28.575) (end 14.4145 28.575) (width 0.38) (layer "B.Cu") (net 2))
 (segment (start 9.398 15.24) (end 9.398 25.146) (width 0.38) (layer "B.Cu") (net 2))
 (segment (start 4.953 16.891) (end 4.953 16.891006) (width 0.38) (layer "B.Cu") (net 2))
 (segment (start 4.318 10.16) (end 8.001 13.843) (width 0.38) (layer "B.Cu") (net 2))
 (segment (start 9.398 25.146) (end 9.398 34.544) (width 0.38) (layer "B.Cu") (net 2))
 (segment (start 22.86 10.16) (end 11.684 10.16) (width 0.38) (layer "B.Cu") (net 2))
 (segment (start 10.553 19.318) (end 7.8745 19.318) (width 0.2) (layer "F.Cu") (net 13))
 (segment (start 10.553 21.451) (end 10.553 19.318) (width 0.2) (layer "F.Cu") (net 13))
 (segment (start 4.953 19.252) (end 3.608 19.252) (width 0.2) (layer "F.Cu") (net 13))
 (segment (start 3.608 19.252) (end 0 22.86) (width 0.2) (layer "F.Cu") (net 13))
 (segment (start 7.727 19.2305) (end 4.9745 19.2305) (width 0.2) (layer "F.Cu") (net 13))
 (segment (start 8.2986 26.7534) (end 8.2986 23.7054) (width 0.2) (layer "F.Cu") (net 13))
 (segment (start 8.2986 23.7054) (end 10.553 21.451) (width 0.2) (layer "F.Cu") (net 13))
 (segment (start 16.383 32.893) (end 16.383 32.512) (width 0.2) (layer "F.Cu") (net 6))
 (segment (start 14.7647 19.2532) (end 16.383 19.2532) (width 0.2) (layer "F.Cu") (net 6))
 (segment (start 20.066 20.066) (end 22.86 22.86) (width 0.2) (layer "F.Cu") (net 6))
 (segment (start 13.7486 33.274) (end 16.002 33.274) (width 0.2) (layer "F.Cu") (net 6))
 (segment (start 16.002 33.274) (end 16.383 32.893) (width 0.2) (layer "F.Cu") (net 6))
 (segment (start 14.6545 19.318) (end 12.253 19.318) (width 0.2) (layer "F.Cu") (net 6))
 (segment (start 20.066 19.252) (end 20.066 20.066) (width 0.2) (layer "F.Cu") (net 6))
 (segment (start 17.6403 19.2532) (end 16.383 19.2532) (width 0.2) (layer "F.Cu") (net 6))
 (segment (start 17.663 19.2305) (end 20.0445 19.2305) (width 0.2) (layer "F.Cu") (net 6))
 (via (at 16.383 19.2532) (size 0.8) (drill 0.4) (layers "F.Cu" "B.Cu") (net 6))
 (via (at 16.383 32.512) (size 0.8) (drill 0.4) (layers "F.Cu" "B.Cu") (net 6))
 (segment (start 16.383 19.2532) (end 16.383 32.512) (width 0.2) (layer "B.Cu") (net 6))
 (segment (start 14.742 17.4055) (end 13.0415 17.4055) (width 0.2) (layer "F.Cu") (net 5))
 (segment (start 11.2886 30.734) (end 10.343301 31.679299) (width 0.2) (layer "F.Cu") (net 5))
 (segment (start 8.7486 33.274) (end 10.343301 31.679299) (width 0.2) (layer "F.Cu") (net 5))
 (segment (start 12.253 17.318) (end 12.953999 17.317999) (width 0.2) (layer "F.Cu") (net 5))
 (segment (start 13.7486 30.734) (end 20.574 30.734) (width 0.2) (layer "F.Cu") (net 5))
 (segment (start 13.7486 30.734) (end 11.2886 30.734) (width 0.2) (layer "F.Cu") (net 5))
 (segment (start 14.742 17.4055) (end 17.663 17.4055) (width 0.2) (layer "F.Cu") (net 5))
 (segment (start 13.0415 17.4055) (end 12.953999 17.317999) (width 0.2) (layer "F.Cu") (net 5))
 (segment (start 20.574 30.734) (end 22.86 33.02) (width 0.2) (layer "F.Cu") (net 5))
 (via (at 10.343301 31.679299) (size 0.8) (drill 0.4) (layers "F.Cu" "B.Cu") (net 5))
 (via (at 12.953999 17.317999) (size 0.8) (drill 0.4) (layers "F.Cu" "B.Cu") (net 5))
 (segment (start 10.3433 19.928698) (end 10.343301 31.679299) (width 0.2) (layer "B.Cu") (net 5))
 (segment (start 12.953999 17.317999) (end 10.3433 19.928698) (width 0.2) (layer "B.Cu") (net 5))
 (segment (start 7.8745 17.318) (end 10.353 17.318) (width 0.2) (layer "F.Cu") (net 11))
 (segment (start 0 17.78) (end 3.048005 17.78) (width 0.2) (layer "F.Cu") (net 11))
 (segment (start 8.2986 30.734) (end 5.207 30.734) (width 0.2) (layer "F.Cu") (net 11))
 (segment (start 6.223005 18.160995) (end 6.477 17.907) (width 0.2) (layer "F.Cu") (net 11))
 (segment (start 6.5324 17.3436) (end 6.477 17.399) (width 0.2) (layer "F.Cu") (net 11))
 (segment (start 3.429 18.160995) (end 6.223005 18.160995) (width 0.2) (layer "F.Cu") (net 11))
 (segment (start 7.7251 17.3436) (end 6.5324 17.3436) (width 0.2) (layer "F.Cu") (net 11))
 (segment (start 6.477 17.907) (end 6.477 17.399) (width 0.2) (layer "F.Cu") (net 11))
 (segment (start 3.048005 17.78) (end 3.429 18.160995) (width 0.2) (layer "F.Cu") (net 11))
 (via (at 5.207 30.734) (size 0.8) (drill 0.4) (layers "F.Cu" "B.Cu") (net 11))
 (via (at 6.477 17.399) (size 0.8) (drill 0.4) (layers "F.Cu" "B.Cu") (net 11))
 (segment (start 5.207 30.734) (end 5.207 18.669) (width 0.2) (layer "B.Cu") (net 11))
 (segment (start 5.207 18.669) (end 6.477 17.399) (width 0.2) (layer "B.Cu") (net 11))
 (segment (start 10.297 27.549) (end 19.441 27.549) (width 0.2) (layer "F.Cu") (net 21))
 (segment (start 9.652 28.194) (end 8.2986 28.194) (width 0.2) (layer "F.Cu") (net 21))
 (segment (start 9.1948 32.004) (end 9.652 31.5468) (width 0.2) (layer "F.Cu") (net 21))
 (segment (start 19.441 27.549) (end 21.59 25.4) (width 0.2) (layer "F.Cu") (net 21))
 (segment (start 8.2986 32.004) (end 9.1948 32.004) (width 0.2) (layer "F.Cu") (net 21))
 (segment (start 9.652 31.5468) (end 9.652 28.194) (width 0.2) (layer "F.Cu") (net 21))
 (segment (start 9.652 28.194) (end 10.297 27.549) (width 0.2) (layer "F.Cu") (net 21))
 (segment (start 21.59 25.4) (end 22.86 25.4) (width 0.2) (layer "F.Cu") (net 21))
 (segment (start 4.689 13.98) (end 4.699 13.97) (width 0.2) (layer "F.Cu") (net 10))
 (segment (start 8.2986 29.464) (end 4.191 29.464) (width 0.2) (layer "F.Cu") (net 10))
 (segment (start 4.0405 13.98) (end 2.784 13.98) (width 0.38) (layer "F.Cu") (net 10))
 (segment (start 2.784 13.98) (end 1.524 15.24) (width 0.38) (layer "F.Cu") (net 10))
 (segment (start 4.0405 13.98) (end 4.689 13.98) (width 0.2) (layer "F.Cu") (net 10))
 (segment (start 1.524 15.24) (end 0 15.24) (width 0.38) (layer "F.Cu") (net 10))
 (via (at 4.191 29.464) (size 0.8) (drill 0.4) (layers "F.Cu" "B.Cu") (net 10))
 (via (at 4.699 13.97) (size 0.8) (drill 0.4) (layers "F.Cu" "B.Cu") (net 10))
 (segment (start 4.699 15.367) (end 4.699 13.97) (width 0.2) (layer "B.Cu") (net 10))
 (segment (start 4.191 15.875) (end 4.699 15.367) (width 0.2) (layer "B.Cu") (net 10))
 (segment (start 4.191 29.464) (end 4.191 15.875) (width 0.2) (layer "B.Cu") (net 10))
 (segment (start 21.844 34.544) (end 22.86 35.56) (width 0.2) (layer "F.Cu") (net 19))
 (segment (start 13.7486 34.544) (end 21.844 34.544) (width 0.2) (layer "F.Cu") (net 19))
 (segment (start 21.844 29.464) (end 22.86 30.48) (width 0.2) (layer "F.Cu") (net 20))
 (segment (start 13.7486 29.464) (end 21.844 29.464) (width 0.2) (layer "F.Cu") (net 20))
 (segment (start 1.524 12.7) (end 0 12.7) (width 0.38) (layer "F.Cu") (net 4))
 (segment (start 2.784 11.44) (end 1.524 12.7) (width 0.38) (layer "F.Cu") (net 4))
 (segment (start 4.0405 11.44) (end 2.784 11.44) (width 0.38) (layer "F.Cu") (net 4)))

